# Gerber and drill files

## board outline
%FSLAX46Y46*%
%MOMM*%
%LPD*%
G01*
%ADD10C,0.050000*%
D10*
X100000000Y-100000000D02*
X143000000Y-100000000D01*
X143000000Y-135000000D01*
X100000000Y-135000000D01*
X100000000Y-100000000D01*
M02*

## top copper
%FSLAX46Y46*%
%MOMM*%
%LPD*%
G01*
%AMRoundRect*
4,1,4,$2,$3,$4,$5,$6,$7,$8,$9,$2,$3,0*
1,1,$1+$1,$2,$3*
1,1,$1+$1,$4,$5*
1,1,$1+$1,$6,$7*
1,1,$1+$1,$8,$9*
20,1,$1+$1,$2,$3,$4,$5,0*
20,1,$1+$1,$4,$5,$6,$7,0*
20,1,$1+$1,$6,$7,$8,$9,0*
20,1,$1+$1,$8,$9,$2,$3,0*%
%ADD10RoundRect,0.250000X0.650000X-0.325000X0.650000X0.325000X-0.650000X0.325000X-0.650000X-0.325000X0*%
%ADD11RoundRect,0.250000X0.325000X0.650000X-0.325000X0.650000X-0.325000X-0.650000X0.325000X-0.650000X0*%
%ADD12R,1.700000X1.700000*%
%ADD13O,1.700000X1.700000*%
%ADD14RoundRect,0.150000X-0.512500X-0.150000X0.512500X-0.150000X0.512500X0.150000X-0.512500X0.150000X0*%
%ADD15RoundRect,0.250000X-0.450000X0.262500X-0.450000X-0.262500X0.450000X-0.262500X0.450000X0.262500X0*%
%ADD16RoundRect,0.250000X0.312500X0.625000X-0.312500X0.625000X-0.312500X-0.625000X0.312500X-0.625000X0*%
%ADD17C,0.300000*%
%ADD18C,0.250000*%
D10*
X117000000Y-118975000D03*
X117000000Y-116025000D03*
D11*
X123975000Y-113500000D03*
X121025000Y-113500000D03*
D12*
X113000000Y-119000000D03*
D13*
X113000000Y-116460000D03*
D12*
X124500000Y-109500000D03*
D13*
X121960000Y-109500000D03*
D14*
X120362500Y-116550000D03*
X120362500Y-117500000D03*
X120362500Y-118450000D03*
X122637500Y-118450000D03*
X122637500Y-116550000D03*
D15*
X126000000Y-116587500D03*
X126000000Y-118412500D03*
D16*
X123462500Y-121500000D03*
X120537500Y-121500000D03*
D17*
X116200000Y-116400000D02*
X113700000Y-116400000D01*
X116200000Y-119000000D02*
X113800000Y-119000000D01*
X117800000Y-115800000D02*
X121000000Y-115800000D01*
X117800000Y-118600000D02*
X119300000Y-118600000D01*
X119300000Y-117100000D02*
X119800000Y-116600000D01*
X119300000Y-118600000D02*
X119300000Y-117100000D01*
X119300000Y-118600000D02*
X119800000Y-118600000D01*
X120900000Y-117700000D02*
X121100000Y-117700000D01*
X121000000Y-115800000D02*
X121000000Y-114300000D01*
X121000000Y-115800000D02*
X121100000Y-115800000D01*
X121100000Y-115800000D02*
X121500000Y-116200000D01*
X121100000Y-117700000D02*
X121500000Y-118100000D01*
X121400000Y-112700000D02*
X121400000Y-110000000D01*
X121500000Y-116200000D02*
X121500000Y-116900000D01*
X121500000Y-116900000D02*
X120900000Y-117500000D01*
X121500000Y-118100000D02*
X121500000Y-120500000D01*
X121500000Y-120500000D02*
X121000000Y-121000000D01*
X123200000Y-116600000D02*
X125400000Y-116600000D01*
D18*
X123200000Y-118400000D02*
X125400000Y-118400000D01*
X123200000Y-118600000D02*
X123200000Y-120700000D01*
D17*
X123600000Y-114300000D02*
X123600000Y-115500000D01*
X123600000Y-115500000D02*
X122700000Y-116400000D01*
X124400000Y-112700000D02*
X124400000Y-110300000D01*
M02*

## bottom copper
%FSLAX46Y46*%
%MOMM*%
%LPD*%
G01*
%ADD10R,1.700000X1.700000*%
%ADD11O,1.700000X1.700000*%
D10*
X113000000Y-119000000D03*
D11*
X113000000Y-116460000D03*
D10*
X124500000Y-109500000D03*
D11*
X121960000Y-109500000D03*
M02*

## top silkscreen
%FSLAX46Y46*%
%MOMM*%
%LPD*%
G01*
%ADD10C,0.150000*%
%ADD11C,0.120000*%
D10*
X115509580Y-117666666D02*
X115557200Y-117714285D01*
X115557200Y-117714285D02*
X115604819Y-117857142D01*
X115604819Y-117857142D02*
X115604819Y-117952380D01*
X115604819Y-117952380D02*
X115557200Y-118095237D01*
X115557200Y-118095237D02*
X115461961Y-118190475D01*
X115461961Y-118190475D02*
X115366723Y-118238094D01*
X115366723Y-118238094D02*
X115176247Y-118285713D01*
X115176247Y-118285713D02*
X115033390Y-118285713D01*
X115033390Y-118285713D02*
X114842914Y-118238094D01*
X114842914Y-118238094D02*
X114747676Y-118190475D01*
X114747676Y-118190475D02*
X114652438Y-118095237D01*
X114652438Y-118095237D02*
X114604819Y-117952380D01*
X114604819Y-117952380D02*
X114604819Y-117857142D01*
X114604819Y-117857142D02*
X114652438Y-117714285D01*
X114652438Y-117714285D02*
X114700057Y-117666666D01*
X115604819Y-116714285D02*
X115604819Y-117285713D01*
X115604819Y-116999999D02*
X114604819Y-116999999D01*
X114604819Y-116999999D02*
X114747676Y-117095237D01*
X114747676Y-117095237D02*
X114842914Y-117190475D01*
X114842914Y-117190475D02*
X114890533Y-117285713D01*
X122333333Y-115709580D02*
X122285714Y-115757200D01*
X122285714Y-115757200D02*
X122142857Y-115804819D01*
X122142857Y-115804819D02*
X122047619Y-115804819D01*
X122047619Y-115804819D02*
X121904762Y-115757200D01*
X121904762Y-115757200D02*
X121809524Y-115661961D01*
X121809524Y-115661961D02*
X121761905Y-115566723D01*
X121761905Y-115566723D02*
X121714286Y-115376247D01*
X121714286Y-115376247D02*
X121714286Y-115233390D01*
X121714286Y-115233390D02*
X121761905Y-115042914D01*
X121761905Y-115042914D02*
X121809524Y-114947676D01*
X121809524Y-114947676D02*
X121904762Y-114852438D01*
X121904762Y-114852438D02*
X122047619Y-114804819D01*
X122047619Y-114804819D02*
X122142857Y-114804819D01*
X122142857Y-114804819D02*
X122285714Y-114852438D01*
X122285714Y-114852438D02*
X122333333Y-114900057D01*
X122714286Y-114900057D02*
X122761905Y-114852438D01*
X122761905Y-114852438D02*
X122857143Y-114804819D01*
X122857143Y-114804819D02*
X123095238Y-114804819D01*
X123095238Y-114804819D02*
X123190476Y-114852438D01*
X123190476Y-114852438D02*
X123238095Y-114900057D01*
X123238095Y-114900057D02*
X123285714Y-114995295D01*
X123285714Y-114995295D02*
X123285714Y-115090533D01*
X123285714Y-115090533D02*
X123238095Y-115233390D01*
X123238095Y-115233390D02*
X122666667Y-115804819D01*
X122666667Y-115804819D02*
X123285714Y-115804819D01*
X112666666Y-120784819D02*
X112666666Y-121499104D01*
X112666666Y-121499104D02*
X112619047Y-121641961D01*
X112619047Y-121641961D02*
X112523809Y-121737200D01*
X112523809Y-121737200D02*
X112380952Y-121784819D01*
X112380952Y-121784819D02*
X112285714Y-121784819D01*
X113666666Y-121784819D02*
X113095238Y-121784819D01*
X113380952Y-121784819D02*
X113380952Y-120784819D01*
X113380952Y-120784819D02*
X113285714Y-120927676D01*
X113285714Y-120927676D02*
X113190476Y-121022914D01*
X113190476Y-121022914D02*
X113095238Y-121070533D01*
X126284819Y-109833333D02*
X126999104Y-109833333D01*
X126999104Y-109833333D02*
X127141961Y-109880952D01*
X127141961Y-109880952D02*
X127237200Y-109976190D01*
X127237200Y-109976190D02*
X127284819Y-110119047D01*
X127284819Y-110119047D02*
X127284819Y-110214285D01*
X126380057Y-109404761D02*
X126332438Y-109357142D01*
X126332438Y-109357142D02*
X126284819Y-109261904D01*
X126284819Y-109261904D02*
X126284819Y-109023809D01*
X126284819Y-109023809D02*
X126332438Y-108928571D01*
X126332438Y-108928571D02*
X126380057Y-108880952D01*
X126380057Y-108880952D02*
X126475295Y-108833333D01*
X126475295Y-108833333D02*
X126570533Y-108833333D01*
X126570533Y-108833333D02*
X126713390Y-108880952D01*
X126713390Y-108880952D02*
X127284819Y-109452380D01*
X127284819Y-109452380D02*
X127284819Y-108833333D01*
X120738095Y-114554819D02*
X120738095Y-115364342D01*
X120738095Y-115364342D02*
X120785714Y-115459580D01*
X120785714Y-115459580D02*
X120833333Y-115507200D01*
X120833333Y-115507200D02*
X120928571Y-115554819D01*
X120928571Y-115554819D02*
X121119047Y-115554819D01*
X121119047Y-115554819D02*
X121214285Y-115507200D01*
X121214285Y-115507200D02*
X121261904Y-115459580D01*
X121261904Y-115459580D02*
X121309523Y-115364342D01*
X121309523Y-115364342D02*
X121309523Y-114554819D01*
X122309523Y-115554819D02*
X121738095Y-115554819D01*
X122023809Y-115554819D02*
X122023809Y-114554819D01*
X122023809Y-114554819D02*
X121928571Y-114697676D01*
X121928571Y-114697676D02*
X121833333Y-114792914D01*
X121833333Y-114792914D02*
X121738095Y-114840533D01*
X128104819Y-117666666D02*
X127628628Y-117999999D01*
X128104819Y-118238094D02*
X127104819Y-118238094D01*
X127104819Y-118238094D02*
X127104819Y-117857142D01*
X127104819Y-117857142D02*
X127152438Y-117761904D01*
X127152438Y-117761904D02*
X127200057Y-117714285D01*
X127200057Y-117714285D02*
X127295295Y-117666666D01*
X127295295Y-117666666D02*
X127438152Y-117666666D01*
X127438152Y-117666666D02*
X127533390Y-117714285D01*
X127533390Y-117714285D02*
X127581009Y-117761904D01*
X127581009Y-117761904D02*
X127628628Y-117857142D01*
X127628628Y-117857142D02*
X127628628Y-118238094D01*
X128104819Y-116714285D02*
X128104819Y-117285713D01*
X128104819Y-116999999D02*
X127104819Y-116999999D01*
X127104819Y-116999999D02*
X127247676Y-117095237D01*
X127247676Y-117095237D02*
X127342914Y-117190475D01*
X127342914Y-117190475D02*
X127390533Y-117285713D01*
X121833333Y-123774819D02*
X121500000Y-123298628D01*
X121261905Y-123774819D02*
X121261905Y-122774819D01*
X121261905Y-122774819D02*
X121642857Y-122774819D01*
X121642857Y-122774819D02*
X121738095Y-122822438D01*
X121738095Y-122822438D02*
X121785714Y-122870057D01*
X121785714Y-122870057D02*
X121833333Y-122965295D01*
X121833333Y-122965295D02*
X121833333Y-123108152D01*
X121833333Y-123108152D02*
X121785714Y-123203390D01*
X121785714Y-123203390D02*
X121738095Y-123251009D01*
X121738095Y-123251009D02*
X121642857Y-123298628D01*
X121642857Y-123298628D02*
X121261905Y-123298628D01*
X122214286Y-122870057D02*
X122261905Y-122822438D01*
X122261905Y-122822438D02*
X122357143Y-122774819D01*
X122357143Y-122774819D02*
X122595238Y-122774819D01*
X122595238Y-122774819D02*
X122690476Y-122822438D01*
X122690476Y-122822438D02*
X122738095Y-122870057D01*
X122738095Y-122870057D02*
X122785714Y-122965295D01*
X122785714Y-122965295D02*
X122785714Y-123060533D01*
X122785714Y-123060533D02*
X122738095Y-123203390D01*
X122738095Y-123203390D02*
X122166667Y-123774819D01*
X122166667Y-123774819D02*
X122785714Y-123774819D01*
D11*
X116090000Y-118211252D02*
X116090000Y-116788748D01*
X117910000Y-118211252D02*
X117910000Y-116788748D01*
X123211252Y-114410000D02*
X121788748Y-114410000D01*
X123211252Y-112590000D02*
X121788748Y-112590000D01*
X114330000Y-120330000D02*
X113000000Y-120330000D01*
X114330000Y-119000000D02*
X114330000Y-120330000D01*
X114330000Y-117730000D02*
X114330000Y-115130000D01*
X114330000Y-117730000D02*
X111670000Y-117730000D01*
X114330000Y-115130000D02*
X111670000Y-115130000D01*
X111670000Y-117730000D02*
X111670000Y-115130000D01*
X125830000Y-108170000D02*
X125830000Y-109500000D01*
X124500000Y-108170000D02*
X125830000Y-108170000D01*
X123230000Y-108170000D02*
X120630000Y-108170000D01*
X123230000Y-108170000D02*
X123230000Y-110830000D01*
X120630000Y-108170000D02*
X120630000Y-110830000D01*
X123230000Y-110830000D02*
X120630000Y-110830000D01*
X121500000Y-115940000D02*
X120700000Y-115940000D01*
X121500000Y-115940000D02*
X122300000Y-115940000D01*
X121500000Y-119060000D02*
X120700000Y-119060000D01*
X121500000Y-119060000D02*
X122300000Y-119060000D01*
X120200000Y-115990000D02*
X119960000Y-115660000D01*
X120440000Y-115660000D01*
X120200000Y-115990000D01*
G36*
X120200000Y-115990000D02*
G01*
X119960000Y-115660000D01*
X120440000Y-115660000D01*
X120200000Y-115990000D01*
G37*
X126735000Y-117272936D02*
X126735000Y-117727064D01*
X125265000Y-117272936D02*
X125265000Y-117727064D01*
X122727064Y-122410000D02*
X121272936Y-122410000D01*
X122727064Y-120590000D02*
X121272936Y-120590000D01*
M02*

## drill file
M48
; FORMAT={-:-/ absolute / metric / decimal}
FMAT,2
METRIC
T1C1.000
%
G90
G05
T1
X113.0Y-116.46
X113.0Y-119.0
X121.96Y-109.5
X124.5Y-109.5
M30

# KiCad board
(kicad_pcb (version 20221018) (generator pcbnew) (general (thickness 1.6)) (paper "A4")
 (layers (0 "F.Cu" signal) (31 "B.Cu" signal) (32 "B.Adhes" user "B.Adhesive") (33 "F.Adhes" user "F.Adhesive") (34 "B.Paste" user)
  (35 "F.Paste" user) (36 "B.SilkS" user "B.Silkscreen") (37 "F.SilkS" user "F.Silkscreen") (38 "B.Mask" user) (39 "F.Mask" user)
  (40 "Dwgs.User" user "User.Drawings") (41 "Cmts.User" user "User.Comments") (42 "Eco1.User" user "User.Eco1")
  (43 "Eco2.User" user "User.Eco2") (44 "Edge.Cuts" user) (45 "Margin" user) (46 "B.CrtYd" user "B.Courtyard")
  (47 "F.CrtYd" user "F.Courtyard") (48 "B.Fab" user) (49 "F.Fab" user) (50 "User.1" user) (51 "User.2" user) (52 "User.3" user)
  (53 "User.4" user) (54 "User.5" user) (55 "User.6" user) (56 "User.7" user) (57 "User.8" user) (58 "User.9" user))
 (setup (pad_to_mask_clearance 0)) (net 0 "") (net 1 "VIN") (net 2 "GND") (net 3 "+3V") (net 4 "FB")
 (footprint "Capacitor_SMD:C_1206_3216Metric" (layer "F.Cu") (at 117 117.5 90)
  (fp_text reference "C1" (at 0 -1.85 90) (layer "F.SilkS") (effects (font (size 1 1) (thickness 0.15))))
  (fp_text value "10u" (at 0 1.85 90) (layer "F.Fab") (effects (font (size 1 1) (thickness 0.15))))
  (fp_line (start -0.711252 -0.91) (end 0.711252 -0.91) (stroke (width 0.12) (type solid)) (layer "F.SilkS"))
  (fp_line (start -0.711252 0.91) (end 0.711252 0.91) (stroke (width 0.12) (type solid)) (layer "F.SilkS"))
  (pad "1" smd roundrect (at -1.475 0 90) (size 1.15 1.8) (layers "F.Cu" "F.Paste" "F.Mask") (roundrect_rratio 0.217391) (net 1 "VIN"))
  (pad "2" smd roundrect (at 1.475 0 90) (size 1.15 1.8) (layers "F.Cu" "F.Paste" "F.Mask") (roundrect_rratio 0.217391) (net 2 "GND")))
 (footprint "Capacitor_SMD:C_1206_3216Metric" (layer "F.Cu") (at 122.5 113.5 180)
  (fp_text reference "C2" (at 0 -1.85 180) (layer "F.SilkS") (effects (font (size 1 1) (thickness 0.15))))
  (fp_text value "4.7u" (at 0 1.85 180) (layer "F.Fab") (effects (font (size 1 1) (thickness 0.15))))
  (fp_line (start -0.711252 -0.91) (end 0.711252 -0.91) (stroke (width 0.12) (type solid)) (layer "F.SilkS"))
  (fp_line (start -0.711252 0.91) (end 0.711252 0.91) (stroke (width 0.12) (type solid)) (layer "F.SilkS"))
  (pad "1" smd roundrect (at -1.475 0 180) (size 1.15 1.8) (layers "F.Cu" "F.Paste" "F.Mask") (roundrect_rratio 0.217391) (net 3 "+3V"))
  (pad "2" smd roundrect (at 1.475 0 180) (size 1.15 1.8) (layers "F.Cu" "F.Paste" "F.Mask") (roundrect_rratio 0.217391) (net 2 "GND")))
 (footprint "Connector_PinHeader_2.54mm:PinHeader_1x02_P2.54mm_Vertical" (layer "F.Cu") (at 113 119 180)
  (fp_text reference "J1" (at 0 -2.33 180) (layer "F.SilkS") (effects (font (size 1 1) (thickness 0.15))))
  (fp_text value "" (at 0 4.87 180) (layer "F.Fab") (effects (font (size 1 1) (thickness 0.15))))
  (fp_line (start -1.33 -1.33) (end 0 -1.33) (stroke (width 0.12) (type solid)) (layer "F.SilkS"))
  (fp_line (start -1.33 0) (end -1.33 -1.33) (stroke (width 0.12) (type solid)) (layer "F.SilkS"))
  (fp_line (start -1.33 1.27) (end -1.33 3.87) (stroke (width 0.12) (type solid)) (layer "F.SilkS"))
  (fp_line (start -1.33 1.27) (end 1.33 1.27) (stroke (width 0.12) (type solid)) (layer "F.SilkS"))
  (fp_line (start -1.33 3.87) (end 1.33 3.87) (stroke (width 0.12) (type solid)) (layer "F.SilkS"))
  (fp_line (start 1.33 1.27) (end 1.33 3.87) (stroke (width 0.12) (type solid)) (layer "F.SilkS"))
  (pad "1" thru_hole rect (at 0 0 180) (size 1.7 1.7) (drill 1) (layers "*.Cu" "*.Mask") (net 1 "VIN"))
  (pad "2" thru_hole oval (at 0 2.54 180) (size 1.7 1.7) (drill 1) (layers "*.Cu" "*.Mask") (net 2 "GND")))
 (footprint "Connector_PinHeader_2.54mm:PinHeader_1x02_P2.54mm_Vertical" (layer "F.Cu") (at 124.5 109.5 -90)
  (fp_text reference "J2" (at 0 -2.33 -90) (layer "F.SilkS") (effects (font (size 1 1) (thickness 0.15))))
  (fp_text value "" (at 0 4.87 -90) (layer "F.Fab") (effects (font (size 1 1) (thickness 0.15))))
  (fp_line (start -1.33 -1.33) (end 0 -1.33) (stroke (width 0.12) (type solid)) (layer "F.SilkS"))
  (fp_line (start -1.33 0) (end -1.33 -1.33) (stroke (width 0.12) (type solid)) (layer "F.SilkS"))
  (fp_line (start -1.33 1.27) (end -1.33 3.87) (stroke (width 0.12) (type solid)) (layer "F.SilkS"))
  (fp_line (start -1.33 1.27) (end 1.33 1.27) (stroke (width 0.12) (type solid)) (layer "F.SilkS"))
  (fp_line (start -1.33 3.87) (end 1.33 3.87) (stroke (width 0.12) (type solid)) (layer "F.SilkS"))
  (fp_line (start 1.33 1.27) (end 1.33 3.87) (stroke (width 0.12) (type solid)) (layer "F.SilkS"))
  (pad "1" thru_hole rect (at 0 0 270) (size 1.7 1.7) (drill 1) (layers "*.Cu" "*.Mask") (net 3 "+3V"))
  (pad "2" thru_hole oval (at 0 2.54 270) (size 1.7 1.7) (drill 1) (layers "*.Cu" "*.Mask") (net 2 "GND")))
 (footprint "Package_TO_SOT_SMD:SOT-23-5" (layer "F.Cu") (at 121.5 117.5)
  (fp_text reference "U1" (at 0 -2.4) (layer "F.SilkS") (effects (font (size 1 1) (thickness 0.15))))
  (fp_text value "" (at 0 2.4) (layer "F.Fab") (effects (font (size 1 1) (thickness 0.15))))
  (fp_line (start 0 -1.56) (end -0.8 -1.56) (stroke (width 0.12) (type solid)) (layer "F.SilkS"))
  (fp_line (start 0 -1.56) (end 0.8 -1.56) (stroke (width 0.12) (type solid)) (layer "F.SilkS"))
  (fp_line (start 0 1.56) (end -0.8 1.56) (stroke (width 0.12) (type solid)) (layer "F.SilkS"))
  (fp_line (start 0 1.56) (end 0.8 1.56) (stroke (width 0.12) (type solid)) (layer "F.SilkS"))
  (fp_poly
   (pts (xy -1.3 -1.51) (xy -1.54 -1.84) (xy -1.06 -1.84) (xy -1.3 -1.51)) (stroke (width 0.12) (type solid)) (fill solid) (layer "F.SilkS"))
  (pad "1" smd roundrect (at -1.1375 -0.95) (size 1.325 0.6) (layers "F.Cu" "F.Paste" "F.Mask") (roundrect_rratio 0.25) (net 1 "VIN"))
  (pad "2" smd roundrect (at -1.1375 0) (size 1.325 0.6) (layers "F.Cu" "F.Paste" "F.Mask") (roundrect_rratio 0.25) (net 2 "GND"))
  (pad "3" smd roundrect (at -1.1375 0.95) (size 1.325 0.6) (layers "F.Cu" "F.Paste" "F.Mask") (roundrect_rratio 0.25) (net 1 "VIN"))
  (pad "4" smd roundrect (at 1.1375 0.95) (size 1.325 0.6) (layers "F.Cu" "F.Paste" "F.Mask") (roundrect_rratio 0.25) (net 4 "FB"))
  (pad "5" smd roundrect (at 1.1375 -0.95) (size 1.325 0.6) (layers "F.Cu" "F.Paste" "F.Mask") (roundrect_rratio 0.25) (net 3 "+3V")))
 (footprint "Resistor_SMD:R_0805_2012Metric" (layer "F.Cu") (at 126 117.5 -90)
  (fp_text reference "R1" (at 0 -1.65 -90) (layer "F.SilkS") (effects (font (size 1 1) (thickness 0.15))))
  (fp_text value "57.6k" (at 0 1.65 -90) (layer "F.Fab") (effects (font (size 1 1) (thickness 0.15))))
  (fp_line (start -0.227064 -0.735) (end 0.227064 -0.735) (stroke (width 0.12) (type solid)) (layer "F.SilkS"))
  (fp_line (start -0.227064 0.735) (end 0.227064 0.735) (stroke (width 0.12) (type solid)) (layer "F.SilkS"))
  (pad "1" smd roundrect (at -0.9125 0 270) (size 1.025 1.4) (layers "F.Cu" "F.Paste" "F.Mask") (roundrect_rratio 0.243902) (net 3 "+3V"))
  (pad "2" smd roundrect (at 0.9125 0 270) (size 1.025 1.4) (layers "F.Cu" "F.Paste" "F.Mask") (roundrect_rratio 0.243902) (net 4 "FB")))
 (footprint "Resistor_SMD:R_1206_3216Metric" (layer "F.Cu") (at 122 121.5 180)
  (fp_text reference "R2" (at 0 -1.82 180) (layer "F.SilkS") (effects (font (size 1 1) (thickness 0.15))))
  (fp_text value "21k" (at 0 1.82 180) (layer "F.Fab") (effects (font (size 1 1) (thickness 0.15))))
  (fp_line (start -0.727064 -0.91) (end 0.727064 -0.91) (stroke (width 0.12) (type solid)) (layer "F.SilkS"))
  (fp_line (start -0.727064 0.91) (end 0.727064 0.91) (stroke (width 0.12) (type solid)) (layer "F.SilkS"))
  (pad "1" smd roundrect (at -1.4625 0 180) (size 1.125 1.75) (layers "F.Cu" "F.Paste" "F.Mask") (roundrect_rratio 0.222222) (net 4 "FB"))
  (pad "2" smd roundrect (at 1.4625 0 180) (size 1.125 1.75) (layers "F.Cu" "F.Paste" "F.Mask") (roundrect_rratio 0.222222) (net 2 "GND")))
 (gr_rect (start 100 100) (end 143 135) (stroke (width 0.05) (type default)) (fill none) (layer "Edge.Cuts"))
 (segment (start 116.2 116.4) (end 113.7 116.4) (width 0.3) (layer "F.Cu") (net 2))
 (segment (start 116.2 119) (end 113.8 119) (width 0.3) (layer "F.Cu") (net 1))
 (segment (start 117.8 115.8) (end 121 115.8) (width 0.3) (layer "F.Cu") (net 2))
 (segment (start 117.8 118.6) (end 119.3 118.6) (width 0.3) (layer "F.Cu") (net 1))
 (segment (start 119.3 117.1) (end 119.8 116.6) (width 0.3) (layer "F.Cu") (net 1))
 (segment (start 119.3 118.6) (end 119.3 117.1) (width 0.3) (layer "F.Cu") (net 1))
 (segment (start 119.3 118.6) (end 119.8 118.6) (width 0.3) (layer "F.Cu") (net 1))
 (segment (start 120.9 117.7) (end 121.1 117.7) (width 0.3) (layer "F.Cu") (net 2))
 (segment (start 121 115.8) (end 121 114.3) (width 0.3) (layer "F.Cu") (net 2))
 (segment (start 121 115.8) (end 121.1 115.8) (width 0.3) (layer "F.Cu") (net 2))
 (segment (start 121.1 115.8) (end 121.5 116.2) (width 0.3) (layer "F.Cu") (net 2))
 (segment (start 121.1 117.7) (end 121.5 118.1) (width 0.3) (layer "F.Cu") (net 2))
 (segment (start 121.4 112.7) (end 121.4 110) (width 0.3) (layer "F.Cu") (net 2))
 (segment (start 121.5 116.2) (end 121.5 116.9) (width 0.3) (layer "F.Cu") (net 2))
 (segment (start 121.5 116.9) (end 120.9 117.5) (width 0.3) (layer "F.Cu") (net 2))
 (segment (start 121.5 118.1) (end 121.5 120.5) (width 0.3) (layer "F.Cu") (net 2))
 (segment (start 121.5 120.5) (end 121 121) (width 0.3) (layer "F.Cu") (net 2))
 (segment (start 123.2 116.6) (end 125.4 116.6) (width 0.3) (layer "F.Cu") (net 3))
 (segment (start 123.2 118.4) (end 125.4 118.4) (width 0.25) (layer "F.Cu") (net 4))
 (segment (start 123.2 118.6) (end 123.2 120.7) (width 0.25) (layer "F.Cu") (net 4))
 (segment (start 123.6 114.3) (end 123.6 115.5) (width 0.3) (layer "F.Cu") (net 3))
 (segment (start 123.6 115.5) (end 122.7 116.4) (width 0.3) (layer "F.Cu") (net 3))
 (segment (start 124.4 112.7) (end 124.4 110.3) (width 0.3) (layer "F.Cu") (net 3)))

